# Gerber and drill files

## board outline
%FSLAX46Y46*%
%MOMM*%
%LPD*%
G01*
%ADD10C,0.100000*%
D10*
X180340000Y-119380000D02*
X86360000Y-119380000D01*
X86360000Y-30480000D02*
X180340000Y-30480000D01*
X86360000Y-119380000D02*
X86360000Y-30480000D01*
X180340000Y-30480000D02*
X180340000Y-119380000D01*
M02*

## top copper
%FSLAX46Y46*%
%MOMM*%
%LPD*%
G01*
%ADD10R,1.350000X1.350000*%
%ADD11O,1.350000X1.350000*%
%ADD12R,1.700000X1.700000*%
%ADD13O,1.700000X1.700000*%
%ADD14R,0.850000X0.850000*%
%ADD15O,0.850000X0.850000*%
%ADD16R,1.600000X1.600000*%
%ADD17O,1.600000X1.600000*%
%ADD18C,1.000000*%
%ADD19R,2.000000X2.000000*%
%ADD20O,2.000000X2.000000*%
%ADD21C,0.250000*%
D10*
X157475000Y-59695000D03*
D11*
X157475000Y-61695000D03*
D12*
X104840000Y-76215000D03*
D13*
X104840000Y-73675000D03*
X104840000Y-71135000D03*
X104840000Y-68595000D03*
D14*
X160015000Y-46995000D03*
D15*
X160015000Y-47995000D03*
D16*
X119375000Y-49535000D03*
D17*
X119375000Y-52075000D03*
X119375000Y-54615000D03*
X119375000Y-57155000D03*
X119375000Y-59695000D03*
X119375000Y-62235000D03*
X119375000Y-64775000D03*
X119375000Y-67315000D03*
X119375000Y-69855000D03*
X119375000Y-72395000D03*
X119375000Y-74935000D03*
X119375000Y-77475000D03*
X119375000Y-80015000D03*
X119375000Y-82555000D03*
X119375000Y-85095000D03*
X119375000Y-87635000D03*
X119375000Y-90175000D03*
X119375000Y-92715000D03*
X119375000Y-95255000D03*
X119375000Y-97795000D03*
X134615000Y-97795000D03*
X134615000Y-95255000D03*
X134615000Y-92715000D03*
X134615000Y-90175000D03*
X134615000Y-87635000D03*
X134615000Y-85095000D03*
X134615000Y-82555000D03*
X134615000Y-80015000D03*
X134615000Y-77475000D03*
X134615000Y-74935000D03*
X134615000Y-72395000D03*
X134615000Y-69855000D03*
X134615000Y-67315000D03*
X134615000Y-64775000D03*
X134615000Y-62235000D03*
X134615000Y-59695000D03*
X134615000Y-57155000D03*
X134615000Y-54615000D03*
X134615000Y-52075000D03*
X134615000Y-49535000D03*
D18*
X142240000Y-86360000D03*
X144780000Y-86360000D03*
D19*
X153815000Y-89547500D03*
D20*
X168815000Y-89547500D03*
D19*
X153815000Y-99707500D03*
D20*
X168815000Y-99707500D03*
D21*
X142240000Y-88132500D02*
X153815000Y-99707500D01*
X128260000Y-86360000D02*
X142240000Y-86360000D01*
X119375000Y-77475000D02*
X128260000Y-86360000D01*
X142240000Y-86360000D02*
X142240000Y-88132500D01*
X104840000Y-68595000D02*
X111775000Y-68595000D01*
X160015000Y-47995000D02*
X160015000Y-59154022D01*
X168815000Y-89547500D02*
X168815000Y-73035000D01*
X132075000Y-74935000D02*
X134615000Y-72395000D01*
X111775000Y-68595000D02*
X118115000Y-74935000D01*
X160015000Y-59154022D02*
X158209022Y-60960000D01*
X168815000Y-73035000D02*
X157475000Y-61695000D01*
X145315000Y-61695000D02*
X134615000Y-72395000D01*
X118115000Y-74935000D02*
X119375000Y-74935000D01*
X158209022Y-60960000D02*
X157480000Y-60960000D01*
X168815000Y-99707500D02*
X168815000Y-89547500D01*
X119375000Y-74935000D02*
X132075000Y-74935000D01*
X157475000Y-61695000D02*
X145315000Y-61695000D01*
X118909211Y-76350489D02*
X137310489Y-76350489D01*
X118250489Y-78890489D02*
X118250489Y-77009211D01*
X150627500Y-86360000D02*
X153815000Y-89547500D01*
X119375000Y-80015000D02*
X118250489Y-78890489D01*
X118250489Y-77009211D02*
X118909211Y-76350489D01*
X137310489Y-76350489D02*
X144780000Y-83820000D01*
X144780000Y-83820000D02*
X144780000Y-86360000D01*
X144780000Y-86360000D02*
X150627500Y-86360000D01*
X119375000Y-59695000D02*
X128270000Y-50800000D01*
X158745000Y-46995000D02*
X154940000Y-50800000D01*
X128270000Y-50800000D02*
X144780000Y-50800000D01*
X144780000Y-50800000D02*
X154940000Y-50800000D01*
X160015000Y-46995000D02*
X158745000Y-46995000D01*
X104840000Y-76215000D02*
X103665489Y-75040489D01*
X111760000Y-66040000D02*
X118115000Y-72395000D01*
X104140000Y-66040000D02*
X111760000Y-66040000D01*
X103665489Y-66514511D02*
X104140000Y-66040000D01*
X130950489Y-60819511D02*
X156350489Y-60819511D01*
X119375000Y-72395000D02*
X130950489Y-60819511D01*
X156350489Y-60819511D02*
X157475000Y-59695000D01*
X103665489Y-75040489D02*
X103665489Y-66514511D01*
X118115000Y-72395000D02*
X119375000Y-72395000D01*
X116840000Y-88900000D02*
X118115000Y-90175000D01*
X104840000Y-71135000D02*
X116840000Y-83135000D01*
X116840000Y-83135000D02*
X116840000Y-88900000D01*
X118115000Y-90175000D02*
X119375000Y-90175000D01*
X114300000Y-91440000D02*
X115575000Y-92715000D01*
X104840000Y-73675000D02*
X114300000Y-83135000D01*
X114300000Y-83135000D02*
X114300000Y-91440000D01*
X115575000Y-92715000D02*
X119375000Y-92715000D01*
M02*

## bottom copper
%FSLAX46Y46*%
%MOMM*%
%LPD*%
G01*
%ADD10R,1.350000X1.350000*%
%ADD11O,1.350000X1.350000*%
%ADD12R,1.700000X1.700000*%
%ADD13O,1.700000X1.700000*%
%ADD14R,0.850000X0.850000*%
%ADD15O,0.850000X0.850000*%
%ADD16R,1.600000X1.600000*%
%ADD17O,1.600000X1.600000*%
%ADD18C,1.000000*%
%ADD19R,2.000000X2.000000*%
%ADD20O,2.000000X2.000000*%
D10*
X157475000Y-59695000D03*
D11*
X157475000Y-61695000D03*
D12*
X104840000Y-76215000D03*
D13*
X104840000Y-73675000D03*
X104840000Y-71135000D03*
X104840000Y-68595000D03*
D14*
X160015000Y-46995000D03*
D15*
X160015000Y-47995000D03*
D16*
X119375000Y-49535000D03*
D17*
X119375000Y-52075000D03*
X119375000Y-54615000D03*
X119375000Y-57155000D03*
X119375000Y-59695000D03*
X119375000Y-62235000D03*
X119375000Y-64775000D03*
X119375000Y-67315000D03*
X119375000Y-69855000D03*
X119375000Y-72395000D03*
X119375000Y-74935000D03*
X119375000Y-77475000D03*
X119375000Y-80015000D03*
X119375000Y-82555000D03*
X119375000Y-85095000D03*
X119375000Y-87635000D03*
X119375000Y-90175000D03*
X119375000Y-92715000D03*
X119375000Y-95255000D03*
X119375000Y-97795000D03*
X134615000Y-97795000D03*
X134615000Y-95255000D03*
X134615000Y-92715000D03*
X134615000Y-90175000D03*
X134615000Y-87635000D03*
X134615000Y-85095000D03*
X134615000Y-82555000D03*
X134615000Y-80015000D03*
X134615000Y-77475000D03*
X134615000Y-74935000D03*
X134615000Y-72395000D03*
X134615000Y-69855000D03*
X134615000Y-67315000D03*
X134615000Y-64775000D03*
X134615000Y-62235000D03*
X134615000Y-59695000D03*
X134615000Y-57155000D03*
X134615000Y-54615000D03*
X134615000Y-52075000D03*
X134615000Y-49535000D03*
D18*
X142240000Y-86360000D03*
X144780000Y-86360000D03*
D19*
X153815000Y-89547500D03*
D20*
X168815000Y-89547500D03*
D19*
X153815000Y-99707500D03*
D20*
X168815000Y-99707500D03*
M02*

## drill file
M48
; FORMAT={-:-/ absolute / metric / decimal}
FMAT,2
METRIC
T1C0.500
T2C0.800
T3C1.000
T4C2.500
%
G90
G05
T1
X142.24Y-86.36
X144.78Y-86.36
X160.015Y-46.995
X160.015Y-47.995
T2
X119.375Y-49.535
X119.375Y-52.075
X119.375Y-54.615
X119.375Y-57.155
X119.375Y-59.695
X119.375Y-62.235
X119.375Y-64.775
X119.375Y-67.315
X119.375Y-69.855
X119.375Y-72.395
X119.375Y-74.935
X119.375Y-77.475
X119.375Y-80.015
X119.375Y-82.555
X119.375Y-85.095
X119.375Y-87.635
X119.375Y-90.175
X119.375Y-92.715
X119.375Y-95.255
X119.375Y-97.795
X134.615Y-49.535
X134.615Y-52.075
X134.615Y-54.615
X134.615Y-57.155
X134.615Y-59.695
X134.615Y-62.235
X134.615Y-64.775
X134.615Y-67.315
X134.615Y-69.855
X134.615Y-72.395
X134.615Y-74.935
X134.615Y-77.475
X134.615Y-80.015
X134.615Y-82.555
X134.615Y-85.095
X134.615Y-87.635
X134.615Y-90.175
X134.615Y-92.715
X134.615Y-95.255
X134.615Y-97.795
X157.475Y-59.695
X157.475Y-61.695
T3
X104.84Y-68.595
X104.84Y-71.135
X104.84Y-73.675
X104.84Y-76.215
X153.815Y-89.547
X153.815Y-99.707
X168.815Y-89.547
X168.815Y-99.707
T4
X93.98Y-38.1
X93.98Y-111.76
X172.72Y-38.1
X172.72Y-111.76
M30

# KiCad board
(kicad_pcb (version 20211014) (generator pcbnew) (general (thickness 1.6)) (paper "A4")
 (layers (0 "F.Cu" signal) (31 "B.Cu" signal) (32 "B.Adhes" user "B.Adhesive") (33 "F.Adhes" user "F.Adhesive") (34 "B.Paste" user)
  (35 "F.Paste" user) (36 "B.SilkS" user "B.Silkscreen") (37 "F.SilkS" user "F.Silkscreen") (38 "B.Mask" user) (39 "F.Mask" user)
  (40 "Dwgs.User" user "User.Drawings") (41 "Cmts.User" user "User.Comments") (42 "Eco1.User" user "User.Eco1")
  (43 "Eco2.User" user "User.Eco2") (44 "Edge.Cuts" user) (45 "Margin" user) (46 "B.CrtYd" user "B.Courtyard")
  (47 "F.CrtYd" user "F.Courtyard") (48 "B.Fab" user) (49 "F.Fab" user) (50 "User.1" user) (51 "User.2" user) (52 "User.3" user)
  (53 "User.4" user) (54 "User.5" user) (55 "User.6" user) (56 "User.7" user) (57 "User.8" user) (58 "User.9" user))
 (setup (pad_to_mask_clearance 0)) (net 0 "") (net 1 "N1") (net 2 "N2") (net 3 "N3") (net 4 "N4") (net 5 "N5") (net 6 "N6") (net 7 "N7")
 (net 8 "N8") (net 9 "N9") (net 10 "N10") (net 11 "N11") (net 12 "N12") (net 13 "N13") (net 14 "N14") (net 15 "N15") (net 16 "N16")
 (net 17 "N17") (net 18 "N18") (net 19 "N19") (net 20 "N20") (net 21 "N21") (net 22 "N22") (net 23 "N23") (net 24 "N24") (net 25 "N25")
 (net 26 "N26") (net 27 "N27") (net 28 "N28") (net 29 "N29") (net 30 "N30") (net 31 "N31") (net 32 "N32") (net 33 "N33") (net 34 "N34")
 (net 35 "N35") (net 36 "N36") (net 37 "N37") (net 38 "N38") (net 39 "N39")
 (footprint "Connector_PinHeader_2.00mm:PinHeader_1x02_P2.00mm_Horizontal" (layer "F.Cu") (at 157.475 59.695)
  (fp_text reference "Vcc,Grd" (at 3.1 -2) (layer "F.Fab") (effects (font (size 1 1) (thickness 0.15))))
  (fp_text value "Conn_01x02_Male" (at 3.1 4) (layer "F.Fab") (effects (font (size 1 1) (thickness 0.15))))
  (pad "1" thru_hole rect (at 0 0) (size 1.35 1.35) (drill 0.8) (layers *.Cu *.Mask) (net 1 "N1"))
  (pad "2" thru_hole oval (at 0 2) (size 1.35 1.35) (drill 0.8) (layers *.Cu *.Mask) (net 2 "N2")))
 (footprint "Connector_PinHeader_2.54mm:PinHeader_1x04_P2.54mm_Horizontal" (layer "F.Cu") (at 104.84 76.215 180)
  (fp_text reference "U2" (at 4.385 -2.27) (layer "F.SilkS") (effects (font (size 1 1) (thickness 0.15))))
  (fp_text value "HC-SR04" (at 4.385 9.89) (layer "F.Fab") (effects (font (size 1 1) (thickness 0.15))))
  (pad "1" thru_hole rect (at 0 0 180) (size 1.7 1.7) (drill 1) (layers *.Cu *.Mask) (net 1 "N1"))
  (pad "2" thru_hole oval (at 0 2.54 180) (size 1.7 1.7) (drill 1) (layers *.Cu *.Mask) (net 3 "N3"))
  (pad "3" thru_hole oval (at 0 5.08 180) (size 1.7 1.7) (drill 1) (layers *.Cu *.Mask) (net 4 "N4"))
  (pad "4" thru_hole oval (at 0 7.62 180) (size 1.7 1.7) (drill 1) (layers *.Cu *.Mask) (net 2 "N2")))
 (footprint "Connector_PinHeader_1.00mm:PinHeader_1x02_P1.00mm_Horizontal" (layer "F.Cu") (at 160.015 46.995)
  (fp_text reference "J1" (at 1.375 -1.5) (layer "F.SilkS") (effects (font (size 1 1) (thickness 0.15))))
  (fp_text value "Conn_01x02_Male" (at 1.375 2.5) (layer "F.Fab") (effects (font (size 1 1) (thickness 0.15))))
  (pad "1" thru_hole rect (at 0 0) (size 0.85 0.85) (drill 0.5) (layers *.Cu *.Mask) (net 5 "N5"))
  (pad "2" thru_hole oval (at 0 1) (size 0.85 0.85) (drill 0.5) (layers *.Cu *.Mask) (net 2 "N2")))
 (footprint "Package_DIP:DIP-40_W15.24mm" (layer "F.Cu") (at 119.375 49.535)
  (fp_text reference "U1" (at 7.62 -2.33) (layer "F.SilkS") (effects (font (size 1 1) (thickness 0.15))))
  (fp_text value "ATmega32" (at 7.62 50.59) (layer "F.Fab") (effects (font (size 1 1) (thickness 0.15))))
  (pad "1" thru_hole rect (at 0 0) (size 1.6 1.6) (drill 0.8) (layers *.Cu *.Mask) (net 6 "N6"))
  (pad "2" thru_hole oval (at 0 2.54) (size 1.6 1.6) (drill 0.8) (layers *.Cu *.Mask) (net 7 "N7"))
  (pad "3" thru_hole oval (at 0 5.08) (size 1.6 1.6) (drill 0.8) (layers *.Cu *.Mask) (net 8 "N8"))
  (pad "4" thru_hole oval (at 0 7.62) (size 1.6 1.6) (drill 0.8) (layers *.Cu *.Mask) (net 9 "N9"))
  (pad "5" thru_hole oval (at 0 10.16) (size 1.6 1.6) (drill 0.8) (layers *.Cu *.Mask) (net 5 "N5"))
  (pad "6" thru_hole oval (at 0 12.7) (size 1.6 1.6) (drill 0.8) (layers *.Cu *.Mask) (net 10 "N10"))
  (pad "7" thru_hole oval (at 0 15.24) (size 1.6 1.6) (drill 0.8) (layers *.Cu *.Mask) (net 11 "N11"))
  (pad "8" thru_hole oval (at 0 17.78) (size 1.6 1.6) (drill 0.8) (layers *.Cu *.Mask) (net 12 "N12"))
  (pad "9" thru_hole oval (at 0 20.32) (size 1.6 1.6) (drill 0.8) (layers *.Cu *.Mask) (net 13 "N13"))
  (pad "10" thru_hole oval (at 0 22.86) (size 1.6 1.6) (drill 0.8) (layers *.Cu *.Mask) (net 1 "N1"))
  (pad "11" thru_hole oval (at 0 25.4) (size 1.6 1.6) (drill 0.8) (layers *.Cu *.Mask) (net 2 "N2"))
  (pad "12" thru_hole oval (at 0 27.94) (size 1.6 1.6) (drill 0.8) (layers *.Cu *.Mask) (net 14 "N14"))
  (pad "13" thru_hole oval (at 0 30.48) (size 1.6 1.6) (drill 0.8) (layers *.Cu *.Mask) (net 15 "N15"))
  (pad "14" thru_hole oval (at 0 33.02) (size 1.6 1.6) (drill 0.8) (layers *.Cu *.Mask) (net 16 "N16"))
  (pad "15" thru_hole oval (at 0 35.56) (size 1.6 1.6) (drill 0.8) (layers *.Cu *.Mask) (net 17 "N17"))
  (pad "16" thru_hole oval (at 0 38.1) (size 1.6 1.6) (drill 0.8) (layers *.Cu *.Mask) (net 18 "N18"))
  (pad "17" thru_hole oval (at 0 40.64) (size 1.6 1.6) (drill 0.8) (layers *.Cu *.Mask) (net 4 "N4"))
  (pad "18" thru_hole oval (at 0 43.18) (size 1.6 1.6) (drill 0.8) (layers *.Cu *.Mask) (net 3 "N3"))
  (pad "19" thru_hole oval (at 0 45.72) (size 1.6 1.6) (drill 0.8) (layers *.Cu *.Mask) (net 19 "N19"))
  (pad "20" thru_hole oval (at 0 48.26) (size 1.6 1.6) (drill 0.8) (layers *.Cu *.Mask) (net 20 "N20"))
  (pad "21" thru_hole oval (at 15.24 48.26) (size 1.6 1.6) (drill 0.8) (layers *.Cu *.Mask) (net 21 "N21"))
  (pad "22" thru_hole oval (at 15.24 45.72) (size 1.6 1.6) (drill 0.8) (layers *.Cu *.Mask) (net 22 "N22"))
  (pad "23" thru_hole oval (at 15.24 43.18) (size 1.6 1.6) (drill 0.8) (layers *.Cu *.Mask) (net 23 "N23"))
  (pad "24" thru_hole oval (at 15.24 40.64) (size 1.6 1.6) (drill 0.8) (layers *.Cu *.Mask) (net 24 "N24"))
  (pad "25" thru_hole oval (at 15.24 38.1) (size 1.6 1.6) (drill 0.8) (layers *.Cu *.Mask) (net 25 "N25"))
  (pad "26" thru_hole oval (at 15.24 35.56) (size 1.6 1.6) (drill 0.8) (layers *.Cu *.Mask) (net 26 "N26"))
  (pad "27" thru_hole oval (at 15.24 33.02) (size 1.6 1.6) (drill 0.8) (layers *.Cu *.Mask) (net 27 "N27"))
  (pad "28" thru_hole oval (at 15.24 30.48) (size 1.6 1.6) (drill 0.8) (layers *.Cu *.Mask) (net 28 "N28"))
  (pad "29" thru_hole oval (at 15.24 27.94) (size 1.6 1.6) (drill 0.8) (layers *.Cu *.Mask) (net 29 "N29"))
  (pad "30" thru_hole oval (at 15.24 25.4) (size 1.6 1.6) (drill 0.8) (layers *.Cu *.Mask) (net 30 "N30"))
  (pad "31" thru_hole oval (at 15.24 22.86) (size 1.6 1.6) (drill 0.8) (layers *.Cu *.Mask) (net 2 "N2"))
  (pad "32" thru_hole oval (at 15.24 20.32) (size 1.6 1.6) (drill 0.8) (layers *.Cu *.Mask) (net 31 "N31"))
  (pad "33" thru_hole oval (at 15.24 17.78) (size 1.6 1.6) (drill 0.8) (layers *.Cu *.Mask) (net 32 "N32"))
  (pad "34" thru_hole oval (at 15.24 15.24) (size 1.6 1.6) (drill 0.8) (layers *.Cu *.Mask) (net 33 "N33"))
  (pad "35" thru_hole oval (at 15.24 12.7) (size 1.6 1.6) (drill 0.8) (layers *.Cu *.Mask) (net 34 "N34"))
  (pad "36" thru_hole oval (at 15.24 10.16) (size 1.6 1.6) (drill 0.8) (layers *.Cu *.Mask) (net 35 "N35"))
  (pad "37" thru_hole oval (at 15.24 7.62) (size 1.6 1.6) (drill 0.8) (layers *.Cu *.Mask) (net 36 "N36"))
  (pad "38" thru_hole oval (at 15.24 5.08) (size 1.6 1.6) (drill 0.8) (layers *.Cu *.Mask) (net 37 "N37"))
  (pad "39" thru_hole oval (at 15.24 2.54) (size 1.6 1.6) (drill 0.8) (layers *.Cu *.Mask) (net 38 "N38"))
  (pad "40" thru_hole oval (at 15.24 0) (size 1.6 1.6) (drill 0.8) (layers *.Cu *.Mask) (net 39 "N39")))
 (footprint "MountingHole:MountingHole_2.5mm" (layer "F.Cu") (at 172.72 38.1)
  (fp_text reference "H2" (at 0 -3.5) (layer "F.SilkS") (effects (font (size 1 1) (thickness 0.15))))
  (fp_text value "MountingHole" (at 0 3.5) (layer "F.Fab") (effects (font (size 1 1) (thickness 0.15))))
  (pad "" np_thru_hole circle (at 0 0) (size 2.5 2.5) (drill 2.5) (layers *.Cu *.Mask)))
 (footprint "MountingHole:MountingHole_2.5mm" (layer "F.Cu") (at 172.72 111.76)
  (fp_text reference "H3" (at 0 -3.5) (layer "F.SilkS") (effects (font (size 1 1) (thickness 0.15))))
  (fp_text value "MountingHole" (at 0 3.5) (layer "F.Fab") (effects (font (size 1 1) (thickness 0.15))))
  (pad "" np_thru_hole circle (at 0 0) (size 2.5 2.5) (drill 2.5) (layers *.Cu *.Mask)))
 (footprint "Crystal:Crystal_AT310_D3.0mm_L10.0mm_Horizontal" (layer "F.Cu") (at 142.24 86.36)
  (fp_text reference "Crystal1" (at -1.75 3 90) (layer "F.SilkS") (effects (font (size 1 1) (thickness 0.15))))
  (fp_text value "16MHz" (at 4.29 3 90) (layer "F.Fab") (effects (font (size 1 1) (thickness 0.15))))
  (pad "1" thru_hole circle (at 0 0) (size 1 1) (drill 0.5) (layers *.Cu *.Mask) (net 14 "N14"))
  (pad "2" thru_hole circle (at 2.54 0) (size 1 1) (drill 0.5) (layers *.Cu *.Mask) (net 15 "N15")))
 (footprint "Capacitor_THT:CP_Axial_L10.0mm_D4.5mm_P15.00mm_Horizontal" (layer "F.Cu") (at 153.815 89.5475)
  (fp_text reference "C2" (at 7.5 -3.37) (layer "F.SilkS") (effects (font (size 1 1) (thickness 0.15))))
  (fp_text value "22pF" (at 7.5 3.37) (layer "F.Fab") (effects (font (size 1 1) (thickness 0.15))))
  (pad "1" thru_hole rect (at 0 0) (size 2 2) (drill 1) (layers *.Cu *.Mask) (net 15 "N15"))
  (pad "2" thru_hole oval (at 15 0) (size 2 2) (drill 1) (layers *.Cu *.Mask) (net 2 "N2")))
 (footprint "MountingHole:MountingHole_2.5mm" (layer "F.Cu") (at 93.98 38.1)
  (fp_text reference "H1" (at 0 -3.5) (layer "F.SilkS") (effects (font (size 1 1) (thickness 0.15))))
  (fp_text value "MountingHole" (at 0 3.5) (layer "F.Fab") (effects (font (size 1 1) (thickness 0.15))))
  (pad "" np_thru_hole circle (at 0 0) (size 2.5 2.5) (drill 2.5) (layers *.Cu *.Mask)))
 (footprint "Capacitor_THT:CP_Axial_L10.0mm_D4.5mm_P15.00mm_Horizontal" (layer "F.Cu") (at 153.815 99.7075)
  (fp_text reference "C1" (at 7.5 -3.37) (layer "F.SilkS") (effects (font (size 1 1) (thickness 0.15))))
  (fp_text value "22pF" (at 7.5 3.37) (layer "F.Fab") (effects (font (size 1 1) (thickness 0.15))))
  (pad "1" thru_hole rect (at 0 0) (size 2 2) (drill 1) (layers *.Cu *.Mask) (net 14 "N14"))
  (pad "2" thru_hole oval (at 15 0) (size 2 2) (drill 1) (layers *.Cu *.Mask) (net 2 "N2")))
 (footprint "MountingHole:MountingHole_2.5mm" (layer "F.Cu") (at 93.98 111.76)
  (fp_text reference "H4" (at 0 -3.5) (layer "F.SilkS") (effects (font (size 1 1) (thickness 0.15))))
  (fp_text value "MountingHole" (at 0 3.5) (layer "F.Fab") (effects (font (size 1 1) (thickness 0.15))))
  (pad "" np_thru_hole circle (at 0 0) (size 2.5 2.5) (drill 2.5) (layers *.Cu *.Mask)))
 (gr_line (start 180.34 119.38) (end 86.36 119.38) (layer "Edge.Cuts") (width 0.1))
 (gr_line (start 86.36 30.48) (end 180.34 30.48) (layer "Edge.Cuts") (width 0.1))
 (gr_line (start 86.36 119.38) (end 86.36 30.48) (layer "Edge.Cuts") (width 0.1))
 (gr_line (start 180.34 30.48) (end 180.34 119.38) (layer "Edge.Cuts") (width 0.1))
 (segment (start 142.24 88.1325) (end 153.815 99.7075) (width 0.25) (layer "F.Cu") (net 14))
 (segment (start 128.26 86.36) (end 142.24 86.36) (width 0.25) (layer "F.Cu") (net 14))
 (segment (start 119.375 77.475) (end 128.26 86.36) (width 0.25) (layer "F.Cu") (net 14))
 (segment (start 142.24 86.36) (end 142.24 88.1325) (width 0.25) (layer "F.Cu") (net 14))
 (segment (start 104.84 68.595) (end 111.775 68.595) (width 0.25) (layer "F.Cu") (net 2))
 (segment (start 160.015 47.995) (end 160.015 59.154022) (width 0.25) (layer "F.Cu") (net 2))
 (segment (start 168.815 89.5475) (end 168.815 73.035) (width 0.25) (layer "F.Cu") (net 2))
 (segment (start 132.075 74.935) (end 134.615 72.395) (width 0.25) (layer "F.Cu") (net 2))
 (segment (start 111.775 68.595) (end 118.115 74.935) (width 0.25) (layer "F.Cu") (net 2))
 (segment (start 160.015 59.154022) (end 158.209022 60.96) (width 0.25) (layer "F.Cu") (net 2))
 (segment (start 168.815 73.035) (end 157.475 61.695) (width 0.25) (layer "F.Cu") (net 2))
 (segment (start 145.315 61.695) (end 134.615 72.395) (width 0.25) (layer "F.Cu") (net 2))
 (segment (start 118.115 74.935) (end 119.375 74.935) (width 0.25) (layer "F.Cu") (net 2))
 (segment (start 158.209022 60.96) (end 157.48 60.96) (width 0.25) (layer "F.Cu") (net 2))
 (segment (start 168.815 99.7075) (end 168.815 89.5475) (width 0.25) (layer "F.Cu") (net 2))
 (segment (start 119.375 74.935) (end 132.075 74.935) (width 0.25) (layer "F.Cu") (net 2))
 (segment (start 157.475 61.695) (end 145.315 61.695) (width 0.25) (layer "F.Cu") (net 2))
 (segment (start 118.909211 76.350489) (end 137.310489 76.350489) (width 0.25) (layer "F.Cu") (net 15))
 (segment (start 118.250489 78.890489) (end 118.250489 77.009211) (width 0.25) (layer "F.Cu") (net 15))
 (segment (start 150.6275 86.36) (end 153.815 89.5475) (width 0.25) (layer "F.Cu") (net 15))
 (segment (start 119.375 80.015) (end 118.250489 78.890489) (width 0.25) (layer "F.Cu") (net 15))
 (segment (start 118.250489 77.009211) (end 118.909211 76.350489) (width 0.25) (layer "F.Cu") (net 15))
 (segment (start 137.310489 76.350489) (end 144.78 83.82) (width 0.25) (layer "F.Cu") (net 15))
 (segment (start 144.78 83.82) (end 144.78 86.36) (width 0.25) (layer "F.Cu") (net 15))
 (segment (start 144.78 86.36) (end 150.6275 86.36) (width 0.25) (layer "F.Cu") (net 15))
 (segment (start 119.375 59.695) (end 128.27 50.8) (width 0.25) (layer "F.Cu") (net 5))
 (segment (start 158.745 46.995) (end 154.94 50.8) (width 0.25) (layer "F.Cu") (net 5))
 (segment (start 128.27 50.8) (end 144.78 50.8) (width 0.25) (layer "F.Cu") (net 5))
 (segment (start 144.78 50.8) (end 154.94 50.8) (width 0.25) (layer "F.Cu") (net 5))
 (segment (start 160.015 46.995) (end 158.745 46.995) (width 0.25) (layer "F.Cu") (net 5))
 (segment (start 104.84 76.215) (end 103.665489 75.040489) (width 0.25) (layer "F.Cu") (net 1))
 (segment (start 111.76 66.04) (end 118.115 72.395) (width 0.25) (layer "F.Cu") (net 1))
 (segment (start 104.14 66.04) (end 111.76 66.04) (width 0.25) (layer "F.Cu") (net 1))
 (segment (start 103.665489 66.514511) (end 104.14 66.04) (width 0.25) (layer "F.Cu") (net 1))
 (segment (start 130.950489 60.819511) (end 156.350489 60.819511) (width 0.25) (layer "F.Cu") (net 1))
 (segment (start 119.375 72.395) (end 130.950489 60.819511) (width 0.25) (layer "F.Cu") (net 1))
 (segment (start 156.350489 60.819511) (end 157.475 59.695) (width 0.25) (layer "F.Cu") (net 1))
 (segment (start 103.665489 75.040489) (end 103.665489 66.514511) (width 0.25) (layer "F.Cu") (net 1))
 (segment (start 118.115 72.395) (end 119.375 72.395) (width 0.25) (layer "F.Cu") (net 1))
 (segment (start 116.84 88.9) (end 118.115 90.175) (width 0.25) (layer "F.Cu") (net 4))
 (segment (start 104.84 71.135) (end 116.84 83.135) (width 0.25) (layer "F.Cu") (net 4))
 (segment (start 116.84 83.135) (end 116.84 88.9) (width 0.25) (layer "F.Cu") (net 4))
 (segment (start 118.115 90.175) (end 119.375 90.175) (width 0.25) (layer "F.Cu") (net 4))
 (segment (start 114.3 91.44) (end 115.575 92.715) (width 0.25) (layer "F.Cu") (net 3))
 (segment (start 104.84 73.675) (end 114.3 83.135) (width 0.25) (layer "F.Cu") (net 3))
 (segment (start 114.3 83.135) (end 114.3 91.44) (width 0.25) (layer "F.Cu") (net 3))
 (segment (start 115.575 92.715) (end 119.375 92.715) (width 0.25) (layer "F.Cu") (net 3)))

